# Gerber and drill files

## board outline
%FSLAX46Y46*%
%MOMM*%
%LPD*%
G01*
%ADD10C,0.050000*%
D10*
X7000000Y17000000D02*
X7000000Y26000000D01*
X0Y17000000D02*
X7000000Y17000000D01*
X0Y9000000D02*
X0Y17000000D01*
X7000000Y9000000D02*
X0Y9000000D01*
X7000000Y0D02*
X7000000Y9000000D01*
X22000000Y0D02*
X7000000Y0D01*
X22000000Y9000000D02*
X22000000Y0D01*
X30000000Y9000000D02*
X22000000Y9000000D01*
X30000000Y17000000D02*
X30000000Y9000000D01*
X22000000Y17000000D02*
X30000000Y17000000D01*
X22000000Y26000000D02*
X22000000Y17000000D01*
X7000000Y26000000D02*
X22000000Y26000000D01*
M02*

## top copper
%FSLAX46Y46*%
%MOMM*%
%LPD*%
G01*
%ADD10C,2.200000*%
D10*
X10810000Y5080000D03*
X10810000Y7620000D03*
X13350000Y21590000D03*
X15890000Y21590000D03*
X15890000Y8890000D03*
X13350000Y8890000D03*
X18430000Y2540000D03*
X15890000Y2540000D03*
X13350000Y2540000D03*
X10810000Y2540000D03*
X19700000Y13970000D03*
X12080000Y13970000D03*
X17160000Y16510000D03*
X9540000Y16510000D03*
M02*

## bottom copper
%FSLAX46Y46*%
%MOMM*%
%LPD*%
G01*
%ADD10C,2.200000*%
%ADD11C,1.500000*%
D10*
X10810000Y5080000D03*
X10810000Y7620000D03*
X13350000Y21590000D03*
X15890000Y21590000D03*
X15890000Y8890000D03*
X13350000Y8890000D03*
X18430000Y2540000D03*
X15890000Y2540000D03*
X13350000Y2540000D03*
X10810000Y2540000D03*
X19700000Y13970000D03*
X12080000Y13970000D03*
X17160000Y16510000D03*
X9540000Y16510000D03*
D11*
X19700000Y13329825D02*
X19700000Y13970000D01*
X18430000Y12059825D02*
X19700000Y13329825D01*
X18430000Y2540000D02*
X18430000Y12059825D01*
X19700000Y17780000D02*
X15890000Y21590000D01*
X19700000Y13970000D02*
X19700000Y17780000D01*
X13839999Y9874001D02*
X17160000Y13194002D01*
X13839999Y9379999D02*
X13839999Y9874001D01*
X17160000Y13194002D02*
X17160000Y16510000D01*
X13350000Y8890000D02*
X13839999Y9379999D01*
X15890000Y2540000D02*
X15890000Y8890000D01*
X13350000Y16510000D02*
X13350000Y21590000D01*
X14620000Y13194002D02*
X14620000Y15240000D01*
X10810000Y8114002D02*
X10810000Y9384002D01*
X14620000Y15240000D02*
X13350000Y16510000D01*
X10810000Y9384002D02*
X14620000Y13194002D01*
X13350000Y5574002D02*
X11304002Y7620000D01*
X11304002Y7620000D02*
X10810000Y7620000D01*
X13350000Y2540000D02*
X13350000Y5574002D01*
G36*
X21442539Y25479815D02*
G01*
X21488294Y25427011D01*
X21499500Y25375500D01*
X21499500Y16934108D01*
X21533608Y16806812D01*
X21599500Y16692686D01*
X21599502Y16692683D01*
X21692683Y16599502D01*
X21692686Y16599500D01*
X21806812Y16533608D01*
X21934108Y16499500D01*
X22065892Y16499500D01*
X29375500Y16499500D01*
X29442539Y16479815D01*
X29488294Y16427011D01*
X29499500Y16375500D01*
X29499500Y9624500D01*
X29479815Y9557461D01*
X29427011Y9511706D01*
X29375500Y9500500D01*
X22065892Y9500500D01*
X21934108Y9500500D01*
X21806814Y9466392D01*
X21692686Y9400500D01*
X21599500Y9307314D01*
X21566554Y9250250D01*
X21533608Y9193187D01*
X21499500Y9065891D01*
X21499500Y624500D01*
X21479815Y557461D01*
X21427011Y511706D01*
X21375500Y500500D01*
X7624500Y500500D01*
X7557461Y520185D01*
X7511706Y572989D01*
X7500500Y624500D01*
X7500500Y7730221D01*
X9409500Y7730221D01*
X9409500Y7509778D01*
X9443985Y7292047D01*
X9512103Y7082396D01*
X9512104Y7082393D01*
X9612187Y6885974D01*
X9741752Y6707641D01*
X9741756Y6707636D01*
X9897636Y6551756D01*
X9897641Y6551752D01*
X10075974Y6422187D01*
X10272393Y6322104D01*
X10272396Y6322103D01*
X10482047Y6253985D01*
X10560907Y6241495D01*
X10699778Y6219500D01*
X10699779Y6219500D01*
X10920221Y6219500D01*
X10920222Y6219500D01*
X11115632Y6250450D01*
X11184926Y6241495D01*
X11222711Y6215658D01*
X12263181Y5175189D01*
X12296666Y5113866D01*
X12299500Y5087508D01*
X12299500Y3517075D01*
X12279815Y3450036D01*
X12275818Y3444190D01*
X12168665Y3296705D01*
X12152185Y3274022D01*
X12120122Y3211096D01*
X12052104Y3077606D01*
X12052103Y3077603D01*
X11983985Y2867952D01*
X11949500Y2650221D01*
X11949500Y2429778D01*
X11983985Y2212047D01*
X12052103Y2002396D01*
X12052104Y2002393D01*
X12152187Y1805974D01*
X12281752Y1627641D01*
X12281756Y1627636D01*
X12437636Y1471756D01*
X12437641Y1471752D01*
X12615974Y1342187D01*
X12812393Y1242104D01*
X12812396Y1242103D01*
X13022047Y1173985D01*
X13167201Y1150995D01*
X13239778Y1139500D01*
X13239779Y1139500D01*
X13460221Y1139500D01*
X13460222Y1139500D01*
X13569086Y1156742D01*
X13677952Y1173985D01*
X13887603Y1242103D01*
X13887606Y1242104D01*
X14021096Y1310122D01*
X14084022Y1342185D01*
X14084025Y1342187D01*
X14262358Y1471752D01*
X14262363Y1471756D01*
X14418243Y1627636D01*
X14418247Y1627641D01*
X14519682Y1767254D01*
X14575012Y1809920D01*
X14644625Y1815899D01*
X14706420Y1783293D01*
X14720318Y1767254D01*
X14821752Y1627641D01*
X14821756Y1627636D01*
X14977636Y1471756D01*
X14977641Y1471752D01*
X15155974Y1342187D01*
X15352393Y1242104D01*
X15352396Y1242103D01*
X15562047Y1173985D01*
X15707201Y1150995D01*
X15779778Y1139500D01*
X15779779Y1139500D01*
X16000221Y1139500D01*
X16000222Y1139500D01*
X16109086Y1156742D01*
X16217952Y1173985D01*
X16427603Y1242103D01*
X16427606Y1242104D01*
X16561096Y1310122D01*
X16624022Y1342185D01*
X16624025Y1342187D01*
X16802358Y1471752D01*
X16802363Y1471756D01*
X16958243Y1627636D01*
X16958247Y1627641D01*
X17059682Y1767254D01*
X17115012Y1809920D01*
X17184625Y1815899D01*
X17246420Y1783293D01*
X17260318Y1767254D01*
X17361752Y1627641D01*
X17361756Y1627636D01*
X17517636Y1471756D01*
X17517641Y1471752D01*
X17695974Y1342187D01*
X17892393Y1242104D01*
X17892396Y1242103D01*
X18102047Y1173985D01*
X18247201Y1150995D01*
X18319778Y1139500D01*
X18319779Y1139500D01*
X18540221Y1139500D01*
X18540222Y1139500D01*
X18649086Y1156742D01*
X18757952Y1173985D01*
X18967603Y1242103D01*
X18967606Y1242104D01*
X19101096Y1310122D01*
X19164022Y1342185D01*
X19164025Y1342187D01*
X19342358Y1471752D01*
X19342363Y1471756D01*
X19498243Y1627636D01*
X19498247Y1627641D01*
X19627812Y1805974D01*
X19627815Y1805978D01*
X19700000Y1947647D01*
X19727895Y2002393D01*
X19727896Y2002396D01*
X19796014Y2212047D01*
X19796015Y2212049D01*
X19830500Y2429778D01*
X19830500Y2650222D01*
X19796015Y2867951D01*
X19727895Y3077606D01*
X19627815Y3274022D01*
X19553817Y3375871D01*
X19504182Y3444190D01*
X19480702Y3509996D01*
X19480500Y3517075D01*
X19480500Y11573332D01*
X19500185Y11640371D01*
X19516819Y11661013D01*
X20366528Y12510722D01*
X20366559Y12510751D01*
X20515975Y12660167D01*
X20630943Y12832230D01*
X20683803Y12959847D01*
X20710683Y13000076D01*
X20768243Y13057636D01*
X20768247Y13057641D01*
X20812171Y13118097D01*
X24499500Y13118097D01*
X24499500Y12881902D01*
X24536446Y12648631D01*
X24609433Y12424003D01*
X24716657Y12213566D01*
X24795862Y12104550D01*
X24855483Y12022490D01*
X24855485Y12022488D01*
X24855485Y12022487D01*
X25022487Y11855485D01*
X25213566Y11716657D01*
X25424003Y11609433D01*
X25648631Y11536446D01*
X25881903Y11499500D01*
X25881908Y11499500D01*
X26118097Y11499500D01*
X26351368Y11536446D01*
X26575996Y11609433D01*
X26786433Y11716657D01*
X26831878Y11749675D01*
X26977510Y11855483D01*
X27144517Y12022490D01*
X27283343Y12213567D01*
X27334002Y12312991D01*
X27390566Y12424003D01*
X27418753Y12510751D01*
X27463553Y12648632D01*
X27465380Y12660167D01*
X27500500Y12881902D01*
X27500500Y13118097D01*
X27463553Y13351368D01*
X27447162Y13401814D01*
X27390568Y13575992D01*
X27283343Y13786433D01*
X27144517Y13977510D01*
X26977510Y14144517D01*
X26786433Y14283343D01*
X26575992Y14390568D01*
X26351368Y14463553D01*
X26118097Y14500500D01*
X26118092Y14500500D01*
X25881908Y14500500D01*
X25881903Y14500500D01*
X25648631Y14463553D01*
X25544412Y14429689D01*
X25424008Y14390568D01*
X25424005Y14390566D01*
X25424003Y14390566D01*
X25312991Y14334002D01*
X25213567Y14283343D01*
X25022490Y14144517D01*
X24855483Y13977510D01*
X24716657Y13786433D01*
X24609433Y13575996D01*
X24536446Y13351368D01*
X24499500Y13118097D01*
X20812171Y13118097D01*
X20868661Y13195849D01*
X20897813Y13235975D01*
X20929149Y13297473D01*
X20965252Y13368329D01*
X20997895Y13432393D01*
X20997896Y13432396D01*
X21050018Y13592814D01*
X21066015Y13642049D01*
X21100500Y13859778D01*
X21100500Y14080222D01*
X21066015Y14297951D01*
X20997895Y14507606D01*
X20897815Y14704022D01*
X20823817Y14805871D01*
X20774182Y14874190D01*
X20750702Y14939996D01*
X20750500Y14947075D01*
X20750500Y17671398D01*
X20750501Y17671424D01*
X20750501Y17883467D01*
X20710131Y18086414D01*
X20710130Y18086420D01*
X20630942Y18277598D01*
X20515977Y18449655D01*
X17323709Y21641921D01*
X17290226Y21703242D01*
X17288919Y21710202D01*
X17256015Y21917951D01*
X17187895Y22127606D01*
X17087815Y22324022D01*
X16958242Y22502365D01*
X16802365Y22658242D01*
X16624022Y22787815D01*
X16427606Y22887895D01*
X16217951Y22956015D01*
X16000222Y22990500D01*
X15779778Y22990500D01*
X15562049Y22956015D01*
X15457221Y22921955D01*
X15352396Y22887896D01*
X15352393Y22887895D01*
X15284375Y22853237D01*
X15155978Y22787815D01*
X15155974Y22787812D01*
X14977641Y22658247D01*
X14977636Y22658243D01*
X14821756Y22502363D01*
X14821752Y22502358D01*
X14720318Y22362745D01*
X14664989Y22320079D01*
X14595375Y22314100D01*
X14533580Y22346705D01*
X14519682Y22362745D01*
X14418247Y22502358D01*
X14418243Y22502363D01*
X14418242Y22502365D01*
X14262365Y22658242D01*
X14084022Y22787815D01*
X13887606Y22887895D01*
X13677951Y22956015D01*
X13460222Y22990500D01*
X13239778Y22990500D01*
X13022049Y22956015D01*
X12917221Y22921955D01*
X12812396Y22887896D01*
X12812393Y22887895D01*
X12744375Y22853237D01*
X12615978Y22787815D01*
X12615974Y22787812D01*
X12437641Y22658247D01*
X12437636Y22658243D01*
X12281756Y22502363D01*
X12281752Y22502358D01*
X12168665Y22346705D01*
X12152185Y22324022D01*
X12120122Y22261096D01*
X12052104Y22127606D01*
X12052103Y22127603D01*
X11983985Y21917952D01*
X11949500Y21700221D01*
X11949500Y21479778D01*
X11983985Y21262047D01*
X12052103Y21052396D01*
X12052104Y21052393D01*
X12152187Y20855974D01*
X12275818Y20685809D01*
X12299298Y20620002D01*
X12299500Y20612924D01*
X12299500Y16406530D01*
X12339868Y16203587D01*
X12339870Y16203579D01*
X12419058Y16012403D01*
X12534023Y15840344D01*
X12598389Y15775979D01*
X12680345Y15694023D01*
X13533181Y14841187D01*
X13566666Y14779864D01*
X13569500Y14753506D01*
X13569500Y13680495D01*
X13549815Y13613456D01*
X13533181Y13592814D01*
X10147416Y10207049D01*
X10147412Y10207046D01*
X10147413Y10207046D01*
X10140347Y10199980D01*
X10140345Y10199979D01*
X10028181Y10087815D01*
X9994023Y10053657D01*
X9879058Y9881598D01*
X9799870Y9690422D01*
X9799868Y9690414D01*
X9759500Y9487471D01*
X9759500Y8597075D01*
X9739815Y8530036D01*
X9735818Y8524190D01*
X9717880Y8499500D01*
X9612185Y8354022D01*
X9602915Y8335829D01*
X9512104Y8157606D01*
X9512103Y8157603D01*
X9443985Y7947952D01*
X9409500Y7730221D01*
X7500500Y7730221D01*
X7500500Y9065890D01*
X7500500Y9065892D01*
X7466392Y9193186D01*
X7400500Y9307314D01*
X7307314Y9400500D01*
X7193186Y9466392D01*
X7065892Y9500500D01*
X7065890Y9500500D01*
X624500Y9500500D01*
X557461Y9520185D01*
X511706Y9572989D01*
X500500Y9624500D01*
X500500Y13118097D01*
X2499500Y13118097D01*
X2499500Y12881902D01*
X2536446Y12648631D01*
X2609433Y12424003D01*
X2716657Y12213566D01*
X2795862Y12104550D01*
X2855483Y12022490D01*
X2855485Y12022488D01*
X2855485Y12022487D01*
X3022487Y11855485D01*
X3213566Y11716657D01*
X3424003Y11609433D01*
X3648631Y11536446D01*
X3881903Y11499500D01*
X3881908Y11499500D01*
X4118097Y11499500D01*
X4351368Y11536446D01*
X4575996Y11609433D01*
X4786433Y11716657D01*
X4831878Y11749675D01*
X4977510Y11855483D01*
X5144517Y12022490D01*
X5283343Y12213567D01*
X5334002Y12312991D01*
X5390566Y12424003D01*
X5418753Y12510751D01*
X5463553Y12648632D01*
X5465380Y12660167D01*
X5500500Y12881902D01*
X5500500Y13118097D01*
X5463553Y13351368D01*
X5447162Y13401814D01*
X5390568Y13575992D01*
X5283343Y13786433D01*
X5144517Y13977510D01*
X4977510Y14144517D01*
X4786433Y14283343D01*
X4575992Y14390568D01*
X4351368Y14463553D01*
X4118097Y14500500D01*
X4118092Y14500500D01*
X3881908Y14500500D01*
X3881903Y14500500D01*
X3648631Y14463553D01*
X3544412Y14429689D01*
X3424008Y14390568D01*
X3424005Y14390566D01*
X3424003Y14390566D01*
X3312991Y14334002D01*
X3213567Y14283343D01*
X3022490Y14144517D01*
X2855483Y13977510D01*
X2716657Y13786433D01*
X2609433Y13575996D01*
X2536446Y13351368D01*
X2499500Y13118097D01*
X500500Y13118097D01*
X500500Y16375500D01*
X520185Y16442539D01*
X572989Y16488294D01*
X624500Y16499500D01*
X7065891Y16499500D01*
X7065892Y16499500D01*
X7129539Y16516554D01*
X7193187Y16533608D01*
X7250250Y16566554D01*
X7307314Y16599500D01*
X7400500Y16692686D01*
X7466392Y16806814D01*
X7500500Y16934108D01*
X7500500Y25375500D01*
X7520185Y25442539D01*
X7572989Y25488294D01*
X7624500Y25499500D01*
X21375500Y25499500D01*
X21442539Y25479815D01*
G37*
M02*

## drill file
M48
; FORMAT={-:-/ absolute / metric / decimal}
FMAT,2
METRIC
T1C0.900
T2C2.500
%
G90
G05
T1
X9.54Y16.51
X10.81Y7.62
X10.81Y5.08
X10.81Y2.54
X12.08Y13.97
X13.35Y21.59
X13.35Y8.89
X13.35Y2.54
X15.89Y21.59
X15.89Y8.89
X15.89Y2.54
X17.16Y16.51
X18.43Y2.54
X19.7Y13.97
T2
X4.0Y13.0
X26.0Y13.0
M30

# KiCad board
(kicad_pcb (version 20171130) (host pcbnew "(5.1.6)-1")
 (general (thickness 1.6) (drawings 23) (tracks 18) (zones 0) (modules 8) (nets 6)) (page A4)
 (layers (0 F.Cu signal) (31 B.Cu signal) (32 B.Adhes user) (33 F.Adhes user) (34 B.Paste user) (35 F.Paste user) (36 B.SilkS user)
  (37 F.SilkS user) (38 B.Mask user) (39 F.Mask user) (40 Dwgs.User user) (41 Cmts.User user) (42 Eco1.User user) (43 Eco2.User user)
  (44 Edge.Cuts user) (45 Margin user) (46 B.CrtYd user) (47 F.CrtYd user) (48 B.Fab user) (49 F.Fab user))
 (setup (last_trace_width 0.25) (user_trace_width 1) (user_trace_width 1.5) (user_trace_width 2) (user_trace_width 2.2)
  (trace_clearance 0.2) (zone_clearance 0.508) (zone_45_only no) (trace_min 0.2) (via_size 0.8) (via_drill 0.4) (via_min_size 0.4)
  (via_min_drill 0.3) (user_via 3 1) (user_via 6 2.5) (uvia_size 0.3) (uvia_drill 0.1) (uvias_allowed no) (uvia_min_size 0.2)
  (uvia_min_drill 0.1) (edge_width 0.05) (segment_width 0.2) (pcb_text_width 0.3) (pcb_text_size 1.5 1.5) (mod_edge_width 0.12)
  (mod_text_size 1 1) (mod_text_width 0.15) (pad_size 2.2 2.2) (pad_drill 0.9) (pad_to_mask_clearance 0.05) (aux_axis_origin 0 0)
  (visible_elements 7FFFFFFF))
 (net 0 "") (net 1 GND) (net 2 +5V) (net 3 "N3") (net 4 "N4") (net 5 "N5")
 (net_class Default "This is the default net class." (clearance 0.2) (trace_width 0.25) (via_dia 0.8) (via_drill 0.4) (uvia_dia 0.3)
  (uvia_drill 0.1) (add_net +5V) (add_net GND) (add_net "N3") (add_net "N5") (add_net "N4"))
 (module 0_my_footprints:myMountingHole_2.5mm (layer F.Cu) (at 4 -13)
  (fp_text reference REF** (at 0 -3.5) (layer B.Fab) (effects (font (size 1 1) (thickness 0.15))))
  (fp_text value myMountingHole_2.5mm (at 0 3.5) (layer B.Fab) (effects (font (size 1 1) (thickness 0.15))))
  (pad 1 np_thru_hole circle (at 0 0) (size 2.5 2.5) (drill 2.5) (layers *.Cu *.Mask)))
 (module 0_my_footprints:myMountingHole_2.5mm (layer F.Cu) (at 26 -13)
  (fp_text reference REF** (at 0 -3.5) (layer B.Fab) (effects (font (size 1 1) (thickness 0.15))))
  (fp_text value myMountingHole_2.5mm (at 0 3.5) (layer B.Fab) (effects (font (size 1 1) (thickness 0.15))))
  (pad 1 np_thru_hole circle (at 0 0) (size 2.5 2.5) (drill 2.5) (layers *.Cu *.Mask)))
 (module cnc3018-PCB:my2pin (layer F.Cu) (at 10.81 -7.62 270)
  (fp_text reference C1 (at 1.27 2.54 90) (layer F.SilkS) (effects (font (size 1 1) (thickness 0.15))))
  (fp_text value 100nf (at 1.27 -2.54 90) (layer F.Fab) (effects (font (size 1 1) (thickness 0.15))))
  (pad 2 thru_hole circle (at 2.54 0 270) (size 2.2 2.2) (drill 0.9) (layers *.Cu *.Mask) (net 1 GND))
  (pad 1 thru_hole circle (at 0 0 270) (size 2.2 2.2) (drill 0.9) (layers *.Cu *.Mask) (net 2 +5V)))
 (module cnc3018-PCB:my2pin (layer F.Cu) (at 13.35 -21.59)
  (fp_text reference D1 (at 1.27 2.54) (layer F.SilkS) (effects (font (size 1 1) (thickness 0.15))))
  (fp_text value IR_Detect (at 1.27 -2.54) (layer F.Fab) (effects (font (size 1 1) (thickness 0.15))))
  (pad 1 thru_hole circle (at 0 0) (size 2.2 2.2) (drill 0.9) (layers *.Cu *.Mask) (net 2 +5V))
  (pad 2 thru_hole circle (at 2.54 0) (size 2.2 2.2) (drill 0.9) (layers *.Cu *.Mask) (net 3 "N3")))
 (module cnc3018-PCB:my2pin (layer F.Cu) (at 13.35 -8.89)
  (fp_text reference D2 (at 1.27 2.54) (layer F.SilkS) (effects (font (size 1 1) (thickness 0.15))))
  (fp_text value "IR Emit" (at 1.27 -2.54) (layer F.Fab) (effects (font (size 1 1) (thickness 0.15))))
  (pad 2 thru_hole circle (at 2.54 0) (size 2.2 2.2) (drill 0.9) (layers *.Cu *.Mask) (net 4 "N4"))
  (pad 1 thru_hole circle (at 0 0) (size 2.2 2.2) (drill 0.9) (layers *.Cu *.Mask) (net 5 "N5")))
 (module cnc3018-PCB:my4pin (layer F.Cu) (at 10.81 -2.54)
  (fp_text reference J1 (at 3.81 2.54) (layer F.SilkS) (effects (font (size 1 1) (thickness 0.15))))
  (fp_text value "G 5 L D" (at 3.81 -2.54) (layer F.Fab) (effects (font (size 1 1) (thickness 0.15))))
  (pad 4 thru_hole circle (at 7.62 0) (size 2.2 2.2) (drill 0.9) (layers *.Cu *.Mask) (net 3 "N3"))
  (pad 3 thru_hole circle (at 5.08 0) (size 2.2 2.2) (drill 0.9) (layers *.Cu *.Mask) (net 4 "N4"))
  (pad 2 thru_hole circle (at 2.54 0) (size 2.2 2.2) (drill 0.9) (layers *.Cu *.Mask) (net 2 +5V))
  (pad 1 thru_hole circle (at 0 0) (size 2.2 2.2) (drill 0.9) (layers *.Cu *.Mask) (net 1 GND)))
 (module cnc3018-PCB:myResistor (layer F.Cu) (at 12.08 -13.97)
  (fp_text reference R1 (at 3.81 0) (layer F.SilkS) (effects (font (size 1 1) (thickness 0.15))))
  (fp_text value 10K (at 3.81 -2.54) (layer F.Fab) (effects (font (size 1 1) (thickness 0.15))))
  (pad 2 thru_hole circle (at 7.62 0) (size 2.2 2.2) (drill 0.9) (layers *.Cu *.Mask) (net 3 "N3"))
  (pad 1 thru_hole circle (at 0 0) (size 2.2 2.2) (drill 0.9) (layers *.Cu *.Mask) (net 1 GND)))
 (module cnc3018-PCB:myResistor (layer F.Cu) (at 17.16 -16.51 180)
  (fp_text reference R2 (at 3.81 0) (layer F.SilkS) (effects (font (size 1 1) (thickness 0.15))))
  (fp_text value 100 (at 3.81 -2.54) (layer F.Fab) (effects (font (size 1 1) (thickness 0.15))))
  (pad 1 thru_hole circle (at 0 0 180) (size 2.2 2.2) (drill 0.9) (layers *.Cu *.Mask) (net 5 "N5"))
  (pad 2 thru_hole circle (at 7.62 0 180) (size 2.2 2.2) (drill 0.9) (layers *.Cu *.Mask) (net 1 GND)))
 (gr_line (start 7 -17) (end 7 -26) (layer Edge.Cuts) (width 0.05))
 (gr_line (start 0 -17) (end 7 -17) (layer Edge.Cuts) (width 0.05))
 (gr_line (start 0 -9) (end 0 -17) (layer Edge.Cuts) (width 0.05))
 (gr_line (start 7 -9) (end 0 -9) (layer Edge.Cuts) (width 0.05))
 (gr_line (start 7 0) (end 7 -9) (layer Edge.Cuts) (width 0.05))
 (gr_line (start 22 0) (end 7 0) (layer Edge.Cuts) (width 0.05))
 (gr_line (start 22 -9) (end 22 0) (layer Edge.Cuts) (width 0.05))
 (gr_line (start 30 -9) (end 22 -9) (layer Edge.Cuts) (width 0.05))
 (gr_line (start 30 -17) (end 30 -9) (layer Edge.Cuts) (width 0.05))
 (gr_line (start 22 -17) (end 30 -17) (layer Edge.Cuts) (width 0.05))
 (gr_line (start 22 -26) (end 22 -17) (layer Edge.Cuts) (width 0.05))
 (gr_line (start 7 -26) (end 22 -26) (layer Edge.Cuts) (width 0.05))
 (segment (start 19.7 -13.329825) (end 19.7 -13.97) (width 1.5) (layer B.Cu) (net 3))
 (segment (start 18.43 -12.059825) (end 19.7 -13.329825) (width 1.5) (layer B.Cu) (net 3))
 (segment (start 18.43 -2.54) (end 18.43 -12.059825) (width 1.5) (layer B.Cu) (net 3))
 (segment (start 19.7 -17.78) (end 15.89 -21.59) (width 1.5) (layer B.Cu) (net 3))
 (segment (start 19.7 -13.97) (end 19.7 -17.78) (width 1.5) (layer B.Cu) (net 3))
 (segment (start 13.839999 -9.874001) (end 17.16 -13.194002) (width 1.5) (layer B.Cu) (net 5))
 (segment (start 13.839999 -9.379999) (end 13.839999 -9.874001) (width 1.5) (layer B.Cu) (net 5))
 (segment (start 17.16 -13.194002) (end 17.16 -16.51) (width 1.5) (layer B.Cu) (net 5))
 (segment (start 13.35 -8.89) (end 13.839999 -9.379999) (width 1.5) (layer B.Cu) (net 5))
 (segment (start 15.89 -2.54) (end 15.89 -8.89) (width 1.5) (layer B.Cu) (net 4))
 (segment (start 13.35 -16.51) (end 13.35 -21.59) (width 1.5) (layer B.Cu) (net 2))
 (segment (start 14.62 -13.194002) (end 14.62 -15.24) (width 1.5) (layer B.Cu) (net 2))
 (segment (start 10.81 -8.114002) (end 10.81 -9.384002) (width 1.5) (layer B.Cu) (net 2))
 (segment (start 14.62 -15.24) (end 13.35 -16.51) (width 1.5) (layer B.Cu) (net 2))
 (segment (start 10.81 -9.384002) (end 14.62 -13.194002) (width 1.5) (layer B.Cu) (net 2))
 (segment (start 13.35 -5.574002) (end 11.304002 -7.62) (width 1.5) (layer B.Cu) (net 2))
 (segment (start 11.304002 -7.62) (end 10.81 -7.62) (width 1.5) (layer B.Cu) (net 2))
 (segment (start 13.35 -2.54) (end 13.35 -5.574002) (width 1.5) (layer B.Cu) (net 2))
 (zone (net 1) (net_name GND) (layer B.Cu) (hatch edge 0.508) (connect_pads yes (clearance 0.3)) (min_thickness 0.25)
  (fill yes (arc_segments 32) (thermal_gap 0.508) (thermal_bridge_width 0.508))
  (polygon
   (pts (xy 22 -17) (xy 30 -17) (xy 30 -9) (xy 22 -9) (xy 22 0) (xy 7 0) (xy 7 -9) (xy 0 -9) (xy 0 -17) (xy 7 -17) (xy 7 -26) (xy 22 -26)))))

